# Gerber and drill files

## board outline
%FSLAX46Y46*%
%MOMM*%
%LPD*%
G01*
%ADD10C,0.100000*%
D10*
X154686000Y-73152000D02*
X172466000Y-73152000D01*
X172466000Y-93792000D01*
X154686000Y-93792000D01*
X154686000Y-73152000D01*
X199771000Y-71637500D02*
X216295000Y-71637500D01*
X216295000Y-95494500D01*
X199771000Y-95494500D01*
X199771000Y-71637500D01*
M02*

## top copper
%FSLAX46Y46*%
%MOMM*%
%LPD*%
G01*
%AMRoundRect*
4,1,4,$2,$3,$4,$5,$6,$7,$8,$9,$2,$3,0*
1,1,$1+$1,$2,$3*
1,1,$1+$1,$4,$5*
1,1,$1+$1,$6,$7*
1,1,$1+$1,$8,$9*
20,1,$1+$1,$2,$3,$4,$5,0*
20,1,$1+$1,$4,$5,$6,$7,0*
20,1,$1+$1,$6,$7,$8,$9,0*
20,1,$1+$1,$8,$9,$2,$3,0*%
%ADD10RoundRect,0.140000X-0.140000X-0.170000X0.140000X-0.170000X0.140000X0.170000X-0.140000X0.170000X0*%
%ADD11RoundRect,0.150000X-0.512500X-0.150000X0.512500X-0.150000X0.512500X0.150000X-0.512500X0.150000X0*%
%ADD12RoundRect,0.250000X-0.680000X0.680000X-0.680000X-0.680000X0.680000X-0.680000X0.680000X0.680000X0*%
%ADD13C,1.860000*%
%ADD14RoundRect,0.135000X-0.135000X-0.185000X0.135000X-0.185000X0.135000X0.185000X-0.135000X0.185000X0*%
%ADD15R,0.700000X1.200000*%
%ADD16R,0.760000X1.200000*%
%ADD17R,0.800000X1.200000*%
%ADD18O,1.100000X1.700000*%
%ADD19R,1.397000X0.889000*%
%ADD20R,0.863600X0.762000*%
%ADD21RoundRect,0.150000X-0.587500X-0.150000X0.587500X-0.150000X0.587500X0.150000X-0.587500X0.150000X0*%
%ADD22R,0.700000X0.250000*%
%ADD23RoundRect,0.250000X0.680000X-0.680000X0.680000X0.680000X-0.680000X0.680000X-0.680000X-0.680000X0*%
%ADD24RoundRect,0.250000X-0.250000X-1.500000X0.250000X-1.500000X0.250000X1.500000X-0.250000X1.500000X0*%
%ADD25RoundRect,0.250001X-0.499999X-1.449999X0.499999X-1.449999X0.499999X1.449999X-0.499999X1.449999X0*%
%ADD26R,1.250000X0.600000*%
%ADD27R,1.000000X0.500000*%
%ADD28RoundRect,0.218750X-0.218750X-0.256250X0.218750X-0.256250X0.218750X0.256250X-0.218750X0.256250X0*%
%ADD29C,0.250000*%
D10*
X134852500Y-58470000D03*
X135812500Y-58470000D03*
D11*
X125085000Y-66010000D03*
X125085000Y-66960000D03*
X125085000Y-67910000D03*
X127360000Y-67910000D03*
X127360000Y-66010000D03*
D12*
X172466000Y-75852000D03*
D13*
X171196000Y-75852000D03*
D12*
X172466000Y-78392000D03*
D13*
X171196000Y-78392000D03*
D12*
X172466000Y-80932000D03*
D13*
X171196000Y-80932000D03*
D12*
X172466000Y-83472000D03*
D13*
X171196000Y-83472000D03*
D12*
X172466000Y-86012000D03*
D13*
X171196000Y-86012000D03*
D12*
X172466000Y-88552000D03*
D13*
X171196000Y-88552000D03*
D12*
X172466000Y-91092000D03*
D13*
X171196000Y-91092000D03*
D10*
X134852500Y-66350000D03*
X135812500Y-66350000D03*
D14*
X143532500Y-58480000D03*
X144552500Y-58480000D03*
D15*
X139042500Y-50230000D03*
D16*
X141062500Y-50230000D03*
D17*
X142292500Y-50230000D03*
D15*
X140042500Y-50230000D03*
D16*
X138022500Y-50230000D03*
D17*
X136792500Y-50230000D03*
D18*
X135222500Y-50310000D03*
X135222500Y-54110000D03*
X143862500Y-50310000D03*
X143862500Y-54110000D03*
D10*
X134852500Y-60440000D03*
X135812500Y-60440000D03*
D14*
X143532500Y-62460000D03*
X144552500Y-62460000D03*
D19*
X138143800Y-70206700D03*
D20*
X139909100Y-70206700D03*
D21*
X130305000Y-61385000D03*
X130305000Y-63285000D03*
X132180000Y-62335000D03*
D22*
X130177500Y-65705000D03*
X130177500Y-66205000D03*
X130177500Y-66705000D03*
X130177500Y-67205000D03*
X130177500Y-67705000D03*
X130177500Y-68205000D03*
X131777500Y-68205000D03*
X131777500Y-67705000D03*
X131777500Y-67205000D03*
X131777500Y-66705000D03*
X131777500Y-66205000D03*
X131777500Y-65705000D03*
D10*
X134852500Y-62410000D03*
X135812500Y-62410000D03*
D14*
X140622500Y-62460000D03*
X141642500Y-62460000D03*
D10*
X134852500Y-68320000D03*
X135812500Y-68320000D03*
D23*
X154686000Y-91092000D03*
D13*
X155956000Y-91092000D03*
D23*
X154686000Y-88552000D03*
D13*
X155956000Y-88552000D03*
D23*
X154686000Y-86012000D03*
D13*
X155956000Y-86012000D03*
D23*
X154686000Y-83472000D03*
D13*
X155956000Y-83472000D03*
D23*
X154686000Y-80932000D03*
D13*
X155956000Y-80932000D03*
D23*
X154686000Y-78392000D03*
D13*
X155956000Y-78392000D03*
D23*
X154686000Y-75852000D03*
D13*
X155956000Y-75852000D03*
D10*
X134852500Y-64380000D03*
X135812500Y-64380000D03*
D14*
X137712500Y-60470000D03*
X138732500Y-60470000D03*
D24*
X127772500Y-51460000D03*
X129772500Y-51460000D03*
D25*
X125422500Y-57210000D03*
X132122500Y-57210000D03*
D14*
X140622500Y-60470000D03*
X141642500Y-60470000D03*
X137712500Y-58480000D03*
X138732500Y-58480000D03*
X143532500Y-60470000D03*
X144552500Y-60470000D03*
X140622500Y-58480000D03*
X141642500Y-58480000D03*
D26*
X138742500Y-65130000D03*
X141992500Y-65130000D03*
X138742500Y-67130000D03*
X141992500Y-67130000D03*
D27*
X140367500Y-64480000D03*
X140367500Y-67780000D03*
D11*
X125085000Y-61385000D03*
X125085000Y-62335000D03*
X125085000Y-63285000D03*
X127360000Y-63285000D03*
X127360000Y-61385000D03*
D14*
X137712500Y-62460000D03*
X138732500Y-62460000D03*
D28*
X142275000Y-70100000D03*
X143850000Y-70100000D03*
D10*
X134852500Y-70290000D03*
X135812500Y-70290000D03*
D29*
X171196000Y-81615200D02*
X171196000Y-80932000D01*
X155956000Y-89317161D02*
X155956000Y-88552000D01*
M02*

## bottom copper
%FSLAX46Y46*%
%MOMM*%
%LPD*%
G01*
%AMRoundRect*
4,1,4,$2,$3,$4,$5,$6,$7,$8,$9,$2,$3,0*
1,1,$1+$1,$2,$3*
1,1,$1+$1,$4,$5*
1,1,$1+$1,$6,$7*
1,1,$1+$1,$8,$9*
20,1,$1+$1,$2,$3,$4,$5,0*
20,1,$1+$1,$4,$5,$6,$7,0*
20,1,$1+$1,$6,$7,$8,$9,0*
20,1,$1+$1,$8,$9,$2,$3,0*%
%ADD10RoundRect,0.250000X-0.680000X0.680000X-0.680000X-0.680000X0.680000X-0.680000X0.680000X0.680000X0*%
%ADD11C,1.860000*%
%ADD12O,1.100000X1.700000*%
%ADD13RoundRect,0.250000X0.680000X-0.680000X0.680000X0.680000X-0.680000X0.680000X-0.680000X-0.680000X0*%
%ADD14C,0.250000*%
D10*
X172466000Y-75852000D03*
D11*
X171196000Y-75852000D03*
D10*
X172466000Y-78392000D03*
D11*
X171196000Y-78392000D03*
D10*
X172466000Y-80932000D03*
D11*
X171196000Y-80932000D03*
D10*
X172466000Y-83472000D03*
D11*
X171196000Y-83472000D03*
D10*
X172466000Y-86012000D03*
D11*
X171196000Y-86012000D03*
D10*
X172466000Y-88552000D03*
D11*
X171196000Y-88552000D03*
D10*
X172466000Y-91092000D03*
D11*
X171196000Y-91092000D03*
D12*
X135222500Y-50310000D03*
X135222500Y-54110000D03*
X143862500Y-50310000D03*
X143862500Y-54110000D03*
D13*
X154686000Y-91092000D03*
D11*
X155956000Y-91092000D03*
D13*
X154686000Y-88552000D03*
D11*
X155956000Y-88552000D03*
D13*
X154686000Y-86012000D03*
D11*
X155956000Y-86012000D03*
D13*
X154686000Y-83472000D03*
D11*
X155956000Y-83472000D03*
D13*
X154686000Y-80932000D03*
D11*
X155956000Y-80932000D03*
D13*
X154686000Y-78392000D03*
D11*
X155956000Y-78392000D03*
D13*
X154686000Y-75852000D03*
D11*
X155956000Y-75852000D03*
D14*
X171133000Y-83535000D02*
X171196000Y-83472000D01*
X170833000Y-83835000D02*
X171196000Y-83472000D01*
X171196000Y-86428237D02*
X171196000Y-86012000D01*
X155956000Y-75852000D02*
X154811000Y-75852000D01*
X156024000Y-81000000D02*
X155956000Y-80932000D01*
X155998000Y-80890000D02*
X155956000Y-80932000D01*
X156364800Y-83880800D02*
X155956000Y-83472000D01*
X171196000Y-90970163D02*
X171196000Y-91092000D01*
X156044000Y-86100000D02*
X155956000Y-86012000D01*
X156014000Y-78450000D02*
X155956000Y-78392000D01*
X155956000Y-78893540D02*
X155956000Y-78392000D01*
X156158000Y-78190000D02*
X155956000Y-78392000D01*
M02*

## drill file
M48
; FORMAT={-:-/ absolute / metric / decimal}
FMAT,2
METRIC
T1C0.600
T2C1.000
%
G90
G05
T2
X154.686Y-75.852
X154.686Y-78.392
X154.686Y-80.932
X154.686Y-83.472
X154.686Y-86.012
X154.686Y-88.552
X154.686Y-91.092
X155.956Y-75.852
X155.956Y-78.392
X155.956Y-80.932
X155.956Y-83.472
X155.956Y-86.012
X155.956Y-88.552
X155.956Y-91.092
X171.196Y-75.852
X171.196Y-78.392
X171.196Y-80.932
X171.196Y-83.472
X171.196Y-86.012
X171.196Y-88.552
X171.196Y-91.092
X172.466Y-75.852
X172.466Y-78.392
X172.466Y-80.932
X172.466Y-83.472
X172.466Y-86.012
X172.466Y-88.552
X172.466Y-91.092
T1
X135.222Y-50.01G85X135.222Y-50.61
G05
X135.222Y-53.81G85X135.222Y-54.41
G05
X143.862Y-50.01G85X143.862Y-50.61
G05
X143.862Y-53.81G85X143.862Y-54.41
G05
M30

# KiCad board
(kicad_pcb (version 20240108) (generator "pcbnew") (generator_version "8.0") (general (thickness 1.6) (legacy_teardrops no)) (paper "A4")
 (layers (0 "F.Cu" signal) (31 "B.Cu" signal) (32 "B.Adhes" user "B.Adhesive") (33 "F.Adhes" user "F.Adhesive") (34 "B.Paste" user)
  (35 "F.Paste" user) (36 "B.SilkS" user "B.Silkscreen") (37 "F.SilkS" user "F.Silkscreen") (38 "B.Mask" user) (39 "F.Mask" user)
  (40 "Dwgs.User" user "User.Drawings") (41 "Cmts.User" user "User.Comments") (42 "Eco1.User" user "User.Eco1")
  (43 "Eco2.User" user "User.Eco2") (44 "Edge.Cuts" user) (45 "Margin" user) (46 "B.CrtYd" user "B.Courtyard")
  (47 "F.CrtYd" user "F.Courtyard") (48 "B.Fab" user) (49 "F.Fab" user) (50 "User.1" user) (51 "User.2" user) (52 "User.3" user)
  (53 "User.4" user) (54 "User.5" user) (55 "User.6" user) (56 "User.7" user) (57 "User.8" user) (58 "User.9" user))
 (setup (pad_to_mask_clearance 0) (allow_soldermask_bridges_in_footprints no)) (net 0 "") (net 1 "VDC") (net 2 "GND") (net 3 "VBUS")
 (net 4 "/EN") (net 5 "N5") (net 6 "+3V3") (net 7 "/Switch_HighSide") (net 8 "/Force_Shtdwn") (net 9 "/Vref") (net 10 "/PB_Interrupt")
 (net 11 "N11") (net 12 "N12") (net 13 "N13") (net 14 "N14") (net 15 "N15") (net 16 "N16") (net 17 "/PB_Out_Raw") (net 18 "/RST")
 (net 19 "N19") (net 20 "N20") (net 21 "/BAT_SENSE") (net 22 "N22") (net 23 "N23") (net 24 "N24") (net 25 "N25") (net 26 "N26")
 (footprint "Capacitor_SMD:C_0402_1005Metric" (layer "F.Cu") (at 135.3325 58.47)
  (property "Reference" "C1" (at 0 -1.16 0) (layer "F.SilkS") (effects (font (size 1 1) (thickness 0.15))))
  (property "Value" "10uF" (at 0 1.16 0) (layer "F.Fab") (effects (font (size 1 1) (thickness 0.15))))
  (pad "1" smd roundrect (at -0.48 0) (size 0.56 0.62) (layers "F.Cu" "F.Paste" "F.Mask") (roundrect_rratio 0.25) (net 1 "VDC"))
  (pad "2" smd roundrect (at 0.48 0) (size 0.56 0.62) (layers "F.Cu" "F.Paste" "F.Mask") (roundrect_rratio 0.25) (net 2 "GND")))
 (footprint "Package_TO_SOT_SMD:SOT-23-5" (layer "F.Cu") (at 126.2225 66.96)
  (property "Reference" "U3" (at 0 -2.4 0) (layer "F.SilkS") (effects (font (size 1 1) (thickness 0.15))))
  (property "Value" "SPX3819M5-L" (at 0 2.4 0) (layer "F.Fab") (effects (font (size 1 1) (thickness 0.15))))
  (pad "1" smd roundrect (at -1.1375 -0.95) (size 1.325 0.6) (layers "F.Cu" "F.Paste" "F.Mask") (roundrect_rratio 0.25) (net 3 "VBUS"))
  (pad "2" smd roundrect (at -1.1375 0) (size 1.325 0.6) (layers "F.Cu" "F.Paste" "F.Mask") (roundrect_rratio 0.25) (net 2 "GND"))
  (pad "3" smd roundrect (at -1.1375 0.95) (size 1.325 0.6) (layers "F.Cu" "F.Paste" "F.Mask") (roundrect_rratio 0.25) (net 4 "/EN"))
  (pad "4" smd roundrect (at 1.1375 0.95) (size 1.325 0.6) (layers "F.Cu" "F.Paste" "F.Mask") (roundrect_rratio 0.25) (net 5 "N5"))
  (pad "5" smd roundrect (at 1.1375 -0.95) (size 1.325 0.6) (layers "F.Cu" "F.Paste" "F.Mask") (roundrect_rratio 0.25) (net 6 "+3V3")))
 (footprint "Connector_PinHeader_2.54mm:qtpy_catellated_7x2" (layer "F.Cu") (at 172.466 73.312 -90)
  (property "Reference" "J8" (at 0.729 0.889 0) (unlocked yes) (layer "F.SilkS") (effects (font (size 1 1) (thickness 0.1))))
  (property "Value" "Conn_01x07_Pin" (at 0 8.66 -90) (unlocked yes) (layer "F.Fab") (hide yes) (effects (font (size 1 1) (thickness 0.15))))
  (pad "1" thru_hole roundrect (at 2.54 0 270) (size 1.86 1.86) (drill 1) (layers "*.Cu" "*.Mask") (remove_unused_layers no)
   (roundrect_rratio 0.1344086022) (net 6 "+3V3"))
  (pad "1" thru_hole circle (at 2.54 1.27 270) (size 1.86 1.86) (drill 1) (layers "*.Cu" "*.Mask") (remove_unused_layers no) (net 6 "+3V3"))
  (pad "2" thru_hole roundrect (at 5.08 0 270) (size 1.86 1.86) (drill 1) (layers "*.Cu" "*.Mask") (remove_unused_layers no)
   (roundrect_rratio 0.1344086022) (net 2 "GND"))
  (pad "2" thru_hole circle (at 5.08 1.27 270) (size 1.86 1.86) (drill 1) (layers "*.Cu" "*.Mask") (remove_unused_layers no) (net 2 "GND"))
  (pad "3" thru_hole roundrect (at 7.62 0 270) (size 1.86 1.86) (drill 1) (layers "*.Cu" "*.Mask") (remove_unused_layers no)
   (roundrect_rratio 0.1344086022) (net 2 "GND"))
  (pad "3" thru_hole circle (at 7.62 1.27 270) (size 1.86 1.86) (drill 1) (layers "*.Cu" "*.Mask") (remove_unused_layers no) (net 2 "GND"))
  (pad "4" thru_hole roundrect (at 10.16 0 270) (size 1.86 1.86) (drill 1) (layers "*.Cu" "*.Mask") (remove_unused_layers no)
   (roundrect_rratio 0.1344086022) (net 2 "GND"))
  (pad "4" thru_hole circle (at 10.16 1.27 270) (size 1.86 1.86) (drill 1) (layers "*.Cu" "*.Mask") (remove_unused_layers no) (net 2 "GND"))
  (pad "5" thru_hole roundrect (at 12.7 0 270) (size 1.86 1.86) (drill 1) (layers "*.Cu" "*.Mask") (remove_unused_layers no)
   (roundrect_rratio 0.1344086022) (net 2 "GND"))
  (pad "5" thru_hole circle (at 12.7 1.27 270) (size 1.86 1.86) (drill 1) (layers "*.Cu" "*.Mask") (remove_unused_layers no) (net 2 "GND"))
  (pad "6" thru_hole roundrect (at 15.24 0 270) (size 1.86 1.86) (drill 1) (layers "*.Cu" "*.Mask") (remove_unused_layers no)
   (roundrect_rratio 0.1344086022) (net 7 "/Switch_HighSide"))
  (pad "6" thru_hole circle (at 15.24 1.27 270) (size 1.86 1.86) (drill 1) (layers "*.Cu" "*.Mask") (remove_unused_layers no)
   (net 7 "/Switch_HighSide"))
  (pad "7" thru_hole roundrect (at 17.78 0 270) (size 1.86 1.86) (drill 1) (layers "*.Cu" "*.Mask") (remove_unused_layers no)
   (roundrect_rratio 0.1344086022) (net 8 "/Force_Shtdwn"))
  (pad "7" thru_hole circle (at 17.78 1.27 270) (size 1.86 1.86) (drill 1) (layers "*.Cu" "*.Mask") (remove_unused_layers no)
   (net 8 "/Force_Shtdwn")))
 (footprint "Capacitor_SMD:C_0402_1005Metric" (layer "F.Cu") (at 135.3325 66.35)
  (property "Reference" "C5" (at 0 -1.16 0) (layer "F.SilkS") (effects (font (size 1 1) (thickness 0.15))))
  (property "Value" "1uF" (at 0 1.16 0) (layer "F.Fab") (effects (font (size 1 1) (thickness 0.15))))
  (pad "1" smd roundrect (at -0.48 0) (size 0.56 0.62) (layers "F.Cu" "F.Paste" "F.Mask") (roundrect_rratio 0.25) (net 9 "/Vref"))
  (pad "2" smd roundrect (at 0.48 0) (size 0.56 0.62) (layers "F.Cu" "F.Paste" "F.Mask") (roundrect_rratio 0.25) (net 2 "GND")))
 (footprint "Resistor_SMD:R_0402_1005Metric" (layer "F.Cu") (at 144.0425 58.48)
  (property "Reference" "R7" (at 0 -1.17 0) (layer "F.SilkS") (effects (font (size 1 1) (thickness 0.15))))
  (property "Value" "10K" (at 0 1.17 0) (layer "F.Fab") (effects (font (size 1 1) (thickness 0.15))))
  (pad "1" smd roundrect (at -0.51 0) (size 0.54 0.64) (layers "F.Cu" "F.Paste" "F.Mask") (roundrect_rratio 0.25) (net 6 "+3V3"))
  (pad "2" smd roundrect (at 0.51 0) (size 0.54 0.64) (layers "F.Cu" "F.Paste" "F.Mask") (roundrect_rratio 0.25) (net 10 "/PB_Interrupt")))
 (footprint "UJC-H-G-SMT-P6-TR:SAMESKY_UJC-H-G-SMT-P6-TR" (layer "F.Cu") (at 139.5425 54.11)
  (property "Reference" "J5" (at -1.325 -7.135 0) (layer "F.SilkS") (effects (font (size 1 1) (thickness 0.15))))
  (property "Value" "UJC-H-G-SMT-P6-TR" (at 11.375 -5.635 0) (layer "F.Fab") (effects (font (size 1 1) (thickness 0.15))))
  (pad "A5" smd rect (at -0.5 -3.88) (size 0.7 1.2) (layers "F.Cu" "F.Paste" "F.Mask") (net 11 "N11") (solder_mask_margin 0.102))
  (pad "A9" smd rect (at 1.52 -3.88) (size 0.76 1.2) (layers "F.Cu" "F.Paste" "F.Mask") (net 3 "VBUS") (solder_mask_margin 0.102))
  (pad "A12" smd rect (at 2.75 -3.88) (size 0.8 1.2) (layers "F.Cu" "F.Paste" "F.Mask") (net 2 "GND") (solder_mask_margin 0.102))
  (pad "B5" smd rect (at 0.5 -3.88) (size 0.7 1.2) (layers "F.Cu" "F.Paste" "F.Mask") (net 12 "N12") (solder_mask_margin 0.102))
  (pad "B9" smd rect (at -1.52 -3.88) (size 0.76 1.2) (layers "F.Cu" "F.Paste" "F.Mask") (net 3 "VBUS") (solder_mask_margin 0.102))
  (pad "B12" smd rect (at -2.75 -3.88) (size 0.8 1.2) (layers "F.Cu" "F.Paste" "F.Mask") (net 2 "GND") (solder_mask_margin 0.102))
  (pad "SH1" thru_hole oval (at -4.32 -3.8) (size 1.1 1.7) (drill oval 0.6 1.2) (layers "*.Cu" "*.Mask") (remove_unused_layers no)
   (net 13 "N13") (solder_mask_margin 0.102))
  (pad "SH2" thru_hole oval (at -4.32 0) (size 1.1 1.7) (drill oval 0.6 1.2) (layers "*.Cu" "*.Mask") (remove_unused_layers no)
   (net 13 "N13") (solder_mask_margin 0.102))
  (pad "SH3" thru_hole oval (at 4.32 -3.8) (size 1.1 1.7) (drill oval 0.6 1.2) (layers "*.Cu" "*.Mask") (remove_unused_layers no)
   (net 13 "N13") (solder_mask_margin 0.102))
  (pad "SH4" thru_hole oval (at 4.32 0) (size 1.1 1.7) (drill oval 0.6 1.2) (layers "*.Cu" "*.Mask") (remove_unused_layers no)
   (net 13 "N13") (solder_mask_margin 0.102)))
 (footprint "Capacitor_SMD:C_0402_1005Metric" (layer "F.Cu") (at 135.3325 60.44)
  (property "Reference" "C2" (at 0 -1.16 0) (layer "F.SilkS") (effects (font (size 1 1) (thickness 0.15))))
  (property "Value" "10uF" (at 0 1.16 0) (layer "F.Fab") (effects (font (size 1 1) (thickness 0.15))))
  (pad "1" smd roundrect (at -0.48 0) (size 0.56 0.62) (layers "F.Cu" "F.Paste" "F.Mask") (roundrect_rratio 0.25) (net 3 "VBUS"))
  (pad "2" smd roundrect (at 0.48 0) (size 0.56 0.62) (layers "F.Cu" "F.Paste" "F.Mask") (roundrect_rratio 0.25) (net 2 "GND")))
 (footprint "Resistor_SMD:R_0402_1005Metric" (layer "F.Cu") (at 144.0425 62.46)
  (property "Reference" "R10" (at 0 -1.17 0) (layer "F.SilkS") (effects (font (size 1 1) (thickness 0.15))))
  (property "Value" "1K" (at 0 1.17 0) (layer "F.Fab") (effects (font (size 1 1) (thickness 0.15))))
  (pad "1" smd roundrect (at -0.51 0) (size 0.54 0.64) (layers "F.Cu" "F.Paste" "F.Mask") (roundrect_rratio 0.25) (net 8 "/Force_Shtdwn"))
  (pad "2" smd roundrect (at 0.51 0) (size 0.54 0.64) (layers "F.Cu" "F.Paste" "F.Mask") (roundrect_rratio 0.25) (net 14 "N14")))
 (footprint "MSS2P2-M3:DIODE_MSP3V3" (layer "F.Cu") (at 138.8931 70.2067)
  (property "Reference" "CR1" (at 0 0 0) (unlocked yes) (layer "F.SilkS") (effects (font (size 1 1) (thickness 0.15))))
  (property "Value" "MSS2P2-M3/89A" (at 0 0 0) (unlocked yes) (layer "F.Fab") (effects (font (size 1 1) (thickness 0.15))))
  (pad "1" smd rect (at -0.7493 0) (size 1.397 0.889) (layers "F.Cu" "F.Paste" "F.Mask") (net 3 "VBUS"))
  (pad "2" smd rect (at 1.016 0) (size 0.8636 0.762) (layers "F.Cu" "F.Paste" "F.Mask") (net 1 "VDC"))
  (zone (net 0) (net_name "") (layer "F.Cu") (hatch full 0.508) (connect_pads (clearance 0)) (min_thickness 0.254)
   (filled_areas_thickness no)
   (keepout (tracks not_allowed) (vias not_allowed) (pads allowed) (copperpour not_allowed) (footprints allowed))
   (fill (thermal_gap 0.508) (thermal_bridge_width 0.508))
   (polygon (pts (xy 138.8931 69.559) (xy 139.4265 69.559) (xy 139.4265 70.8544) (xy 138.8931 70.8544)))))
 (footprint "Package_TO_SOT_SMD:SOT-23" (layer "F.Cu") (at 131.2425 62.335)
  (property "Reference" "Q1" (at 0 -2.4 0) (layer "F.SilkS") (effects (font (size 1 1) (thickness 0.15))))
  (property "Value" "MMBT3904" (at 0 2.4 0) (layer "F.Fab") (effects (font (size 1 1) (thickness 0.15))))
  (pad "1" smd roundrect (at -0.9375 -0.95) (size 1.475 0.6) (layers "F.Cu" "F.Paste" "F.Mask") (roundrect_rratio 0.25) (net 14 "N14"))
  (pad "2" smd roundrect (at -0.9375 0.95) (size 1.475 0.6) (layers "F.Cu" "F.Paste" "F.Mask") (roundrect_rratio 0.25) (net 2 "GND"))
  (pad "3" smd roundrect (at 0.9375 0) (size 1.475 0.6) (layers "F.Cu" "F.Paste" "F.Mask") (roundrect_rratio 0.25)
   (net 7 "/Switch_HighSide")))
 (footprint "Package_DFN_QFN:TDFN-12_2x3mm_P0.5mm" (layer "F.Cu") (at 130.9775 66.955)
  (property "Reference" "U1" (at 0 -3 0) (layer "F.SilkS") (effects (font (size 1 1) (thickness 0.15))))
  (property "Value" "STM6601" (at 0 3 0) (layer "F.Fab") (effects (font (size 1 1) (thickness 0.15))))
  (pad "1" smd rect (at -0.8 -1.25) (size 0.7 0.25) (layers "F.Cu" "F.Paste" "F.Mask") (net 3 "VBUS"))
  (pad "2" smd rect (at -0.8 -0.75) (size 0.7 0.25) (layers "F.Cu" "F.Paste" "F.Mask") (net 7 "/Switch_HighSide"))
  (pad "3" smd rect (at -0.8 -0.25) (size 0.7 0.25) (layers "F.Cu" "F.Paste" "F.Mask") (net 9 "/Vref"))
  (pad "4" smd rect (at -0.8 0.25) (size 0.7 0.25) (layers "F.Cu" "F.Paste" "F.Mask") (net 6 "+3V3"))
  (pad "5" smd rect (at -0.8 0.75) (size 0.7 0.25) (layers "F.Cu" "F.Paste" "F.Mask") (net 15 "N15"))
  (pad "6" smd rect (at -0.8 1.25) (size 0.7 0.25) (layers "F.Cu" "F.Paste" "F.Mask") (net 7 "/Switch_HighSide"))
  (pad "7" smd rect (at 0.8 1.25) (size 0.7 0.25) (layers "F.Cu" "F.Paste" "F.Mask") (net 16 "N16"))
  (pad "8" smd rect (at 0.8 0.75) (size 0.7 0.25) (layers "F.Cu" "F.Paste" "F.Mask") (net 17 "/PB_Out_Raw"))
  (pad "9" smd rect (at 0.8 0.25) (size 0.7 0.25) (layers "F.Cu" "F.Paste" "F.Mask") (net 4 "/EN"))
  (pad "10" smd rect (at 0.8 -0.25) (size 0.7 0.25) (layers "F.Cu" "F.Paste" "F.Mask") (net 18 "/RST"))
  (pad "11" smd rect (at 0.8 -0.75) (size 0.7 0.25) (layers "F.Cu" "F.Paste" "F.Mask") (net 10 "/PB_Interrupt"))
  (pad "12" smd rect (at 0.8 -1.25) (size 0.7 0.25) (layers "F.Cu" "F.Paste" "F.Mask") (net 2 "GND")))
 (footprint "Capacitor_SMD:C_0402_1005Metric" (layer "F.Cu") (at 135.3325 62.41)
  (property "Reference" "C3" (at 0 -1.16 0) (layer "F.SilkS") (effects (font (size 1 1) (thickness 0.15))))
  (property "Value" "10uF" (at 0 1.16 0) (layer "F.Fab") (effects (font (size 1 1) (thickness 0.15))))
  (pad "1" smd roundrect (at -0.48 0) (size 0.56 0.62) (layers "F.Cu" "F.Paste" "F.Mask") (roundrect_rratio 0.25) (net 6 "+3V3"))
  (pad "2" smd roundrect (at 0.48 0) (size 0.56 0.62) (layers "F.Cu" "F.Paste" "F.Mask") (roundrect_rratio 0.25) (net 2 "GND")))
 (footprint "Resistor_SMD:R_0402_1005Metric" (layer "F.Cu") (at 141.1325 62.46)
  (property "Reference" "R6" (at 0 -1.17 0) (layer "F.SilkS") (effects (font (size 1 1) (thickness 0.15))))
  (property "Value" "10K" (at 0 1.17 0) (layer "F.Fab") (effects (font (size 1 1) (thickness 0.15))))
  (pad "1" smd roundrect (at -0.51 0) (size 0.54 0.64) (layers "F.Cu" "F.Paste" "F.Mask") (roundrect_rratio 0.25) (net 6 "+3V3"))
  (pad "2" smd roundrect (at 0.51 0) (size 0.54 0.64) (layers "F.Cu" "F.Paste" "F.Mask") (roundrect_rratio 0.25) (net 18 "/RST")))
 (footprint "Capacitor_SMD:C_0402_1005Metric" (layer "F.Cu") (at 135.3325 68.32)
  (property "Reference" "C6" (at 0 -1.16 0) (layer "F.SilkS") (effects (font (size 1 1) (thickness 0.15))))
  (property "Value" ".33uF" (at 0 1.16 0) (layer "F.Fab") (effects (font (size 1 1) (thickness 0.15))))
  (pad "1" smd roundrect (at -0.48 0) (size 0.56 0.62) (layers "F.Cu" "F.Paste" "F.Mask") (roundrect_rratio 0.25) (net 15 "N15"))
  (pad "2" smd roundrect (at 0.48 0) (size 0.56 0.62) (layers "F.Cu" "F.Paste" "F.Mask") (roundrect_rratio 0.25) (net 2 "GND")))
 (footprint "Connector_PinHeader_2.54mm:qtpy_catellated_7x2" (layer "F.Cu") (at 154.686 93.632 90)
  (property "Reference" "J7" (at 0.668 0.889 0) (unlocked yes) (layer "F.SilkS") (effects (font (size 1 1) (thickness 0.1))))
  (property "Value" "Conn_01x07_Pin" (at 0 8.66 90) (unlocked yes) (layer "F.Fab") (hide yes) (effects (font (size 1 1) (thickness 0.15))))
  (pad "1" thru_hole roundrect (at 2.54 0 90) (size 1.86 1.86) (drill 1) (layers "*.Cu" "*.Mask") (remove_unused_layers no)
   (roundrect_rratio 0.1344086022) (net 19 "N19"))
  (pad "1" thru_hole circle (at 2.54 1.27 90) (size 1.86 1.86) (drill 1) (layers "*.Cu" "*.Mask") (remove_unused_layers no) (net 19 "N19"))
  (pad "2" thru_hole roundrect (at 5.08 0 90) (size 1.86 1.86) (drill 1) (layers "*.Cu" "*.Mask") (remove_unused_layers no)
   (roundrect_rratio 0.1344086022) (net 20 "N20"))
  (pad "2" thru_hole circle (at 5.08 1.27 90) (size 1.86 1.86) (drill 1) (layers "*.Cu" "*.Mask") (remove_unused_layers no) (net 20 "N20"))
  (pad "3" thru_hole roundrect (at 7.62 0 90) (size 1.86 1.86) (drill 1) (layers "*.Cu" "*.Mask") (remove_unused_layers no)
   (roundrect_rratio 0.1344086022) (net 17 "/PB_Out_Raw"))
  (pad "3" thru_hole circle (at 7.62 1.27 90) (size 1.86 1.86) (drill 1) (layers "*.Cu" "*.Mask") (remove_unused_layers no)
   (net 17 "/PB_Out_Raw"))
  (pad "4" thru_hole roundrect (at 10.16 0 90) (size 1.86 1.86) (drill 1) (layers "*.Cu" "*.Mask") (remove_unused_layers no)
   (roundrect_rratio 0.1344086022) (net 4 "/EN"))
  (pad "4" thru_hole circle (at 10.16 1.27 90) (size 1.86 1.86) (drill 1) (layers "*.Cu" "*.Mask") (remove_unused_layers no) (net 4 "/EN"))
  (pad "5" thru_hole roundrect (at 12.7 0 90) (size 1.86 1.86) (drill 1) (layers "*.Cu" "*.Mask") (remove_unused_layers no)
   (roundrect_rratio 0.1344086022) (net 18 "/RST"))
  (pad "5" thru_hole circle (at 12.7 1.27 90) (size 1.86 1.86) (drill 1) (layers "*.Cu" "*.Mask") (remove_unused_layers no) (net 18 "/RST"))
  (pad "6" thru_hole roundrect (at 15.24 0 90) (size 1.86 1.86) (drill 1) (layers "*.Cu" "*.Mask") (remove_unused_layers no)
   (roundrect_rratio 0.1344086022) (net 10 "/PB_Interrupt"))
  (pad "6" thru_hole circle (at 15.24 1.27 90) (size 1.86 1.86) (drill 1) (layers "*.Cu" "*.Mask") (remove_unused_layers no)
   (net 10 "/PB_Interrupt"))
  (pad "7" thru_hole roundrect (at 17.78 0 90) (size 1.86 1.86) (drill 1) (layers "*.Cu" "*.Mask") (remove_unused_layers no)
   (roundrect_rratio 0.1344086022) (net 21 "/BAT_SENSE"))
  (pad "7" thru_hole circle (at 17.78 1.27 90) (size 1.86 1.86) (drill 1) (layers "*.Cu" "*.Mask") (remove_unused_layers no)
   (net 21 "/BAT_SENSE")))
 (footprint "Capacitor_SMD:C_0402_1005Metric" (layer "F.Cu") (at 135.3325 64.38)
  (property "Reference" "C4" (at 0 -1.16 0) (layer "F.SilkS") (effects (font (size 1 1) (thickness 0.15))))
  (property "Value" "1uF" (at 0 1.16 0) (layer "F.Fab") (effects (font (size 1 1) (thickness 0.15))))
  (pad "1" smd roundrect (at -0.48 0) (size 0.56 0.62) (layers "F.Cu" "F.Paste" "F.Mask") (roundrect_rratio 0.25) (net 6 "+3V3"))
  (pad "2" smd roundrect (at 0.48 0) (size 0.56 0.62) (layers "F.Cu" "F.Paste" "F.Mask") (roundrect_rratio 0.25) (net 2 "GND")))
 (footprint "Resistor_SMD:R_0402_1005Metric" (layer "F.Cu") (at 138.2225 60.47)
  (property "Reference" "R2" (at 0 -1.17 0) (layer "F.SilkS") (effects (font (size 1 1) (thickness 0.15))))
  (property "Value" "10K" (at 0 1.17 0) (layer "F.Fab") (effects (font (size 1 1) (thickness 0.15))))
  (pad "1" smd roundrect (at -0.51 0) (size 0.54 0.64) (layers "F.Cu" "F.Paste" "F.Mask") (roundrect_rratio 0.25) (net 2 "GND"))
  (pad "2" smd roundrect (at 0.51 0) (size 0.54 0.64) (layers "F.Cu" "F.Paste" "F.Mask") (roundrect_rratio 0.25) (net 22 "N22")))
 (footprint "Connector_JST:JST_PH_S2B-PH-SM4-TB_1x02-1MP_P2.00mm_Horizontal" (layer "F.Cu") (at 128.7725 54.31)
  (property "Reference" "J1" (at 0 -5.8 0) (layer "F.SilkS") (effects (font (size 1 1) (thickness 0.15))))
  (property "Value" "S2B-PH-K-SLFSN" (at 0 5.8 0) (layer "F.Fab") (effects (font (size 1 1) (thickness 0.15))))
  (pad "1" smd roundrect (at -1 -2.85) (size 1 3.5) (layers "F.Cu" "F.Paste" "F.Mask") (roundrect_rratio 0.25) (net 1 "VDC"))
  (pad "2" smd roundrect (at 1 -2.85) (size 1 3.5) (layers "F.Cu" "F.Paste" "F.Mask") (roundrect_rratio 0.25) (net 2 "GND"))
  (pad "MP" smd roundrect (at -3.35 2.9) (size 1.5 3.4) (layers "F.Cu" "F.Paste" "F.Mask") (roundrect_rratio 0.166667))
  (pad "MP" smd roundrect (at 3.35 2.9) (size 1.5 3.4) (layers "F.Cu" "F.Paste" "F.Mask") (roundrect_rratio 0.166667)))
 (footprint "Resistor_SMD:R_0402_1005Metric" (layer "F.Cu") (at 141.1325 60.47)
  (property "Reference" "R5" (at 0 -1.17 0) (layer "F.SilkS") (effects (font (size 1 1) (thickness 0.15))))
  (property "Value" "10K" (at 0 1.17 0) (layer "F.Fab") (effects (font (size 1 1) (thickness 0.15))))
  (pad "1" smd roundrect (at -0.51 0) (size 0.54 0.64) (layers "F.Cu" "F.Paste" "F.Mask") (roundrect_rratio 0.25) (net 6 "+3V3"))
  (pad "2" smd roundrect (at 0.51 0) (size 0.54 0.64) (layers "F.Cu" "F.Paste" "F.Mask") (roundrect_rratio 0.25) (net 17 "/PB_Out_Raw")))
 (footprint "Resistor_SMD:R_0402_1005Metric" (layer "F.Cu") (at 138.2225 58.48)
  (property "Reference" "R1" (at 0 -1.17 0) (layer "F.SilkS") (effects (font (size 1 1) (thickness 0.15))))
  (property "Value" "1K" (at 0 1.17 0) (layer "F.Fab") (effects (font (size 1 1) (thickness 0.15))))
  (pad "1" smd roundrect (at -0.51 0) (size 0.54 0.64) (layers "F.Cu" "F.Paste" "F.Mask") (roundrect_rratio 0.25) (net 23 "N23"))
  (pad "2" smd roundrect (at 0.51 0) (size 0.54 0.64) (layers "F.Cu" "F.Paste" "F.Mask") (roundrect_rratio 0.25) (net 3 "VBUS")))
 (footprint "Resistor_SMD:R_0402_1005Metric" (layer "F.Cu") (at 144.0425 60.47)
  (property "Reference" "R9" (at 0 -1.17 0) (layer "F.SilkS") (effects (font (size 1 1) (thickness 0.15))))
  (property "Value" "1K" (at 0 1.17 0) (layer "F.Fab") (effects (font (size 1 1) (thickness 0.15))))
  (pad "1" smd roundrect (at -0.51 0) (size 0.54 0.64) (layers "F.Cu" "F.Paste" "F.Mask") (roundrect_rratio 0.25) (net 3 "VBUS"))
  (pad "2" smd roundrect (at 0.51 0) (size 0.54 0.64) (layers "F.Cu" "F.Paste" "F.Mask") (roundrect_rratio 0.25) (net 16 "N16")))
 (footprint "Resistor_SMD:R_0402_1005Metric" (layer "F.Cu") (at 141.1325 58.48)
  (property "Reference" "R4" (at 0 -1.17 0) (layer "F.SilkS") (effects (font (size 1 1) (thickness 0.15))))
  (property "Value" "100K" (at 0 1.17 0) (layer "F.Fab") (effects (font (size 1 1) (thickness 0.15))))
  (pad "1" smd roundrect (at -0.51 0) (size 0.54 0.64) (layers "F.Cu" "F.Paste" "F.Mask") (roundrect_rratio 0.25) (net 21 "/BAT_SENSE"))
  (pad "2" smd roundrect (at 0.51 0) (size 0.54 0.64) (layers "F.Cu" "F.Paste" "F.Mask") (roundrect_rratio 0.25) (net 2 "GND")))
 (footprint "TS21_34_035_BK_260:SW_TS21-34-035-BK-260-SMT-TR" (layer "F.Cu") (at 140.3675 66.13)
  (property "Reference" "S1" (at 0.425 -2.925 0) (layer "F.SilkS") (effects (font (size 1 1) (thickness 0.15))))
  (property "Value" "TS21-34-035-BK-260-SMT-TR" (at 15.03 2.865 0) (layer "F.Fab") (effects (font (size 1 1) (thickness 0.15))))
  (pad "1" smd rect (at -1.625 -1) (size 1.25 0.6) (layers "F.Cu" "F.Paste" "F.Mask") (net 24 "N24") (solder_mask_margin 0.102))
  (pad "2" smd rect (at 1.625 -1) (size 1.25 0.6) (layers "F.Cu" "F.Paste" "F.Mask") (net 2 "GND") (solder_mask_margin 0.102))
  (pad "3" smd rect (at -1.625 1) (size 1.25 0.6) (layers "F.Cu" "F.Paste" "F.Mask") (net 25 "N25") (solder_mask_margin 0.102))
  (pad "4" smd rect (at 1.625 1) (size 1.25 0.6) (layers "F.Cu" "F.Paste" "F.Mask") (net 7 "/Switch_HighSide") (solder_mask_margin 0.102))
  (pad "SH1" smd rect (at 0 -1.65) (size 1 0.5) (layers "F.Cu" "F.Paste" "F.Mask") (solder_mask_margin 0.102))
  (pad "SH2" smd rect (at 0 1.65) (size 1 0.5) (layers "F.Cu" "F.Paste" "F.Mask") (solder_mask_margin 0.102)))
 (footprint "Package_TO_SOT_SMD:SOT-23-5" (layer "F.Cu") (at 126.2225 62.335)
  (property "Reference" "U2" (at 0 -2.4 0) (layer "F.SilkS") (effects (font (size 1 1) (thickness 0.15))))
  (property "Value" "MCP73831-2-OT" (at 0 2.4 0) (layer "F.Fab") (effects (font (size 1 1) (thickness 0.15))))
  (pad "1" smd roundrect (at -1.1375 -0.95) (size 1.325 0.6) (layers "F.Cu" "F.Paste" "F.Mask") (roundrect_rratio 0.25) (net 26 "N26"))
  (pad "2" smd roundrect (at -1.1375 0) (size 1.325 0.6) (layers "F.Cu" "F.Paste" "F.Mask") (roundrect_rratio 0.25) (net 2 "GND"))
  (pad "3" smd roundrect (at -1.1375 0.95) (size 1.325 0.6) (layers "F.Cu" "F.Paste" "F.Mask") (roundrect_rratio 0.25) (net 1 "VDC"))
  (pad "4" smd roundrect (at 1.1375 0.95) (size 1.325 0.6) (layers "F.Cu" "F.Paste" "F.Mask") (roundrect_rratio 0.25) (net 3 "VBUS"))
  (pad "5" smd roundrect (at 1.1375 -0.95) (size 1.325 0.6) (layers "F.Cu" "F.Paste" "F.Mask") (roundrect_rratio 0.25) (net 22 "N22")))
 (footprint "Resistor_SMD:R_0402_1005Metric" (layer "F.Cu") (at 138.2225 62.46)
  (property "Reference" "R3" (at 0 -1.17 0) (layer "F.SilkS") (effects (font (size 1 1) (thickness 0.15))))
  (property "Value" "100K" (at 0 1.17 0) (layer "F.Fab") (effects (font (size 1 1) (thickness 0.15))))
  (pad "1" smd roundrect (at -0.51 0) (size 0.54 0.64) (layers "F.Cu" "F.Paste" "F.Mask") (roundrect_rratio 0.25) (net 1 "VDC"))
  (pad "2" smd roundrect (at 0.51 0) (size 0.54 0.64) (layers "F.Cu" "F.Paste" "F.Mask") (roundrect_rratio 0.25) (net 21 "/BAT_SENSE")))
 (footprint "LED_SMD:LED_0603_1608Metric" (layer "F.Cu") (at 143.0625 70.1)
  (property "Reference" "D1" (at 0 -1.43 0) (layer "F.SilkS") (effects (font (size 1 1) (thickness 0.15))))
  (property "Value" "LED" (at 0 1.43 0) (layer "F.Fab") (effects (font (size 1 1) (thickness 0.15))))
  (pad "1" smd roundrect (at -0.7875 0) (size 0.875 0.95) (layers "F.Cu" "F.Paste" "F.Mask") (roundrect_rratio 0.25) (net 26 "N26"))
  (pad "2" smd roundrect (at 0.7875 0) (size 0.875 0.95) (layers "F.Cu" "F.Paste" "F.Mask") (roundrect_rratio 0.25) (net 23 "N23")))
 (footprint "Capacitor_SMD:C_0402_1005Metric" (layer "F.Cu") (at 135.3325 70.29)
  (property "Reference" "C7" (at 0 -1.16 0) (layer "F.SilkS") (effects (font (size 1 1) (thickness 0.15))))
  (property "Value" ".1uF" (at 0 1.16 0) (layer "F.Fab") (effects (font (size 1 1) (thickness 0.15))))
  (pad "1" smd roundrect (at -0.48 0) (size 0.56 0.62) (layers "F.Cu" "F.Paste" "F.Mask") (roundrect_rratio 0.25) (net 3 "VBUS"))
  (pad "2" smd roundrect (at 0.48 0) (size 0.56 0.62) (layers "F.Cu" "F.Paste" "F.Mask") (roundrect_rratio 0.25) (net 2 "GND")))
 (gr_rect (start 154.686 73.152) (end 172.466 93.792) (stroke (width 0.1) (type default)) (fill none) (layer "Edge.Cuts"))
 (gr_rect (start 199.771 71.6375) (end 216.295 95.4945) (stroke (width 0.1) (type default)) (fill none) (layer "Edge.Cuts"))
 (segment (start 171.196 81.6152) (end 171.196 80.932) (width 0.25) (layer "F.Cu") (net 2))
 (segment (start 171.133 83.535) (end 171.196 83.472) (width 0.25) (layer "B.Cu") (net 2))
 (segment (start 170.833 83.835) (end 171.196 83.472) (width 0.25) (layer "B.Cu") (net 2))
 (segment (start 171.196 86.428237) (end 171.196 86.012) (width 0.25) (layer "B.Cu") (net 2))
 (segment (start 155.956 75.852) (end 154.811 75.852) (width 0.25) (layer "B.Cu") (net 21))
 (segment (start 156.024 81) (end 155.956 80.932) (width 0.25) (layer "B.Cu") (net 18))
 (segment (start 155.998 80.89) (end 155.956 80.932) (width 0.25) (layer "B.Cu") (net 18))
 (segment (start 156.3648 83.8808) (end 155.956 83.472) (width 0.25) (layer "B.Cu") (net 4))
 (segment (start 171.196 90.970163) (end 171.196 91.092) (width 0.25) (layer "B.Cu") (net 8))
 (segment (start 156.044 86.1) (end 155.956 86.012) (width 0.25) (layer "B.Cu") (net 17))
 (segment (start 156.014 78.45) (end 155.956 78.392) (width 0.25) (layer "B.Cu") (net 10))
 (segment (start 155.956 78.89354) (end 155.956 78.392) (width 0.25) (layer "B.Cu") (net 10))
 (segment (start 156.158 78.19) (end 155.956 78.392) (width 0.25) (layer "B.Cu") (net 10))
 (segment (start 155.956 89.317161) (end 155.956 88.552) (width 0.25) (layer "F.Cu") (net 20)))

